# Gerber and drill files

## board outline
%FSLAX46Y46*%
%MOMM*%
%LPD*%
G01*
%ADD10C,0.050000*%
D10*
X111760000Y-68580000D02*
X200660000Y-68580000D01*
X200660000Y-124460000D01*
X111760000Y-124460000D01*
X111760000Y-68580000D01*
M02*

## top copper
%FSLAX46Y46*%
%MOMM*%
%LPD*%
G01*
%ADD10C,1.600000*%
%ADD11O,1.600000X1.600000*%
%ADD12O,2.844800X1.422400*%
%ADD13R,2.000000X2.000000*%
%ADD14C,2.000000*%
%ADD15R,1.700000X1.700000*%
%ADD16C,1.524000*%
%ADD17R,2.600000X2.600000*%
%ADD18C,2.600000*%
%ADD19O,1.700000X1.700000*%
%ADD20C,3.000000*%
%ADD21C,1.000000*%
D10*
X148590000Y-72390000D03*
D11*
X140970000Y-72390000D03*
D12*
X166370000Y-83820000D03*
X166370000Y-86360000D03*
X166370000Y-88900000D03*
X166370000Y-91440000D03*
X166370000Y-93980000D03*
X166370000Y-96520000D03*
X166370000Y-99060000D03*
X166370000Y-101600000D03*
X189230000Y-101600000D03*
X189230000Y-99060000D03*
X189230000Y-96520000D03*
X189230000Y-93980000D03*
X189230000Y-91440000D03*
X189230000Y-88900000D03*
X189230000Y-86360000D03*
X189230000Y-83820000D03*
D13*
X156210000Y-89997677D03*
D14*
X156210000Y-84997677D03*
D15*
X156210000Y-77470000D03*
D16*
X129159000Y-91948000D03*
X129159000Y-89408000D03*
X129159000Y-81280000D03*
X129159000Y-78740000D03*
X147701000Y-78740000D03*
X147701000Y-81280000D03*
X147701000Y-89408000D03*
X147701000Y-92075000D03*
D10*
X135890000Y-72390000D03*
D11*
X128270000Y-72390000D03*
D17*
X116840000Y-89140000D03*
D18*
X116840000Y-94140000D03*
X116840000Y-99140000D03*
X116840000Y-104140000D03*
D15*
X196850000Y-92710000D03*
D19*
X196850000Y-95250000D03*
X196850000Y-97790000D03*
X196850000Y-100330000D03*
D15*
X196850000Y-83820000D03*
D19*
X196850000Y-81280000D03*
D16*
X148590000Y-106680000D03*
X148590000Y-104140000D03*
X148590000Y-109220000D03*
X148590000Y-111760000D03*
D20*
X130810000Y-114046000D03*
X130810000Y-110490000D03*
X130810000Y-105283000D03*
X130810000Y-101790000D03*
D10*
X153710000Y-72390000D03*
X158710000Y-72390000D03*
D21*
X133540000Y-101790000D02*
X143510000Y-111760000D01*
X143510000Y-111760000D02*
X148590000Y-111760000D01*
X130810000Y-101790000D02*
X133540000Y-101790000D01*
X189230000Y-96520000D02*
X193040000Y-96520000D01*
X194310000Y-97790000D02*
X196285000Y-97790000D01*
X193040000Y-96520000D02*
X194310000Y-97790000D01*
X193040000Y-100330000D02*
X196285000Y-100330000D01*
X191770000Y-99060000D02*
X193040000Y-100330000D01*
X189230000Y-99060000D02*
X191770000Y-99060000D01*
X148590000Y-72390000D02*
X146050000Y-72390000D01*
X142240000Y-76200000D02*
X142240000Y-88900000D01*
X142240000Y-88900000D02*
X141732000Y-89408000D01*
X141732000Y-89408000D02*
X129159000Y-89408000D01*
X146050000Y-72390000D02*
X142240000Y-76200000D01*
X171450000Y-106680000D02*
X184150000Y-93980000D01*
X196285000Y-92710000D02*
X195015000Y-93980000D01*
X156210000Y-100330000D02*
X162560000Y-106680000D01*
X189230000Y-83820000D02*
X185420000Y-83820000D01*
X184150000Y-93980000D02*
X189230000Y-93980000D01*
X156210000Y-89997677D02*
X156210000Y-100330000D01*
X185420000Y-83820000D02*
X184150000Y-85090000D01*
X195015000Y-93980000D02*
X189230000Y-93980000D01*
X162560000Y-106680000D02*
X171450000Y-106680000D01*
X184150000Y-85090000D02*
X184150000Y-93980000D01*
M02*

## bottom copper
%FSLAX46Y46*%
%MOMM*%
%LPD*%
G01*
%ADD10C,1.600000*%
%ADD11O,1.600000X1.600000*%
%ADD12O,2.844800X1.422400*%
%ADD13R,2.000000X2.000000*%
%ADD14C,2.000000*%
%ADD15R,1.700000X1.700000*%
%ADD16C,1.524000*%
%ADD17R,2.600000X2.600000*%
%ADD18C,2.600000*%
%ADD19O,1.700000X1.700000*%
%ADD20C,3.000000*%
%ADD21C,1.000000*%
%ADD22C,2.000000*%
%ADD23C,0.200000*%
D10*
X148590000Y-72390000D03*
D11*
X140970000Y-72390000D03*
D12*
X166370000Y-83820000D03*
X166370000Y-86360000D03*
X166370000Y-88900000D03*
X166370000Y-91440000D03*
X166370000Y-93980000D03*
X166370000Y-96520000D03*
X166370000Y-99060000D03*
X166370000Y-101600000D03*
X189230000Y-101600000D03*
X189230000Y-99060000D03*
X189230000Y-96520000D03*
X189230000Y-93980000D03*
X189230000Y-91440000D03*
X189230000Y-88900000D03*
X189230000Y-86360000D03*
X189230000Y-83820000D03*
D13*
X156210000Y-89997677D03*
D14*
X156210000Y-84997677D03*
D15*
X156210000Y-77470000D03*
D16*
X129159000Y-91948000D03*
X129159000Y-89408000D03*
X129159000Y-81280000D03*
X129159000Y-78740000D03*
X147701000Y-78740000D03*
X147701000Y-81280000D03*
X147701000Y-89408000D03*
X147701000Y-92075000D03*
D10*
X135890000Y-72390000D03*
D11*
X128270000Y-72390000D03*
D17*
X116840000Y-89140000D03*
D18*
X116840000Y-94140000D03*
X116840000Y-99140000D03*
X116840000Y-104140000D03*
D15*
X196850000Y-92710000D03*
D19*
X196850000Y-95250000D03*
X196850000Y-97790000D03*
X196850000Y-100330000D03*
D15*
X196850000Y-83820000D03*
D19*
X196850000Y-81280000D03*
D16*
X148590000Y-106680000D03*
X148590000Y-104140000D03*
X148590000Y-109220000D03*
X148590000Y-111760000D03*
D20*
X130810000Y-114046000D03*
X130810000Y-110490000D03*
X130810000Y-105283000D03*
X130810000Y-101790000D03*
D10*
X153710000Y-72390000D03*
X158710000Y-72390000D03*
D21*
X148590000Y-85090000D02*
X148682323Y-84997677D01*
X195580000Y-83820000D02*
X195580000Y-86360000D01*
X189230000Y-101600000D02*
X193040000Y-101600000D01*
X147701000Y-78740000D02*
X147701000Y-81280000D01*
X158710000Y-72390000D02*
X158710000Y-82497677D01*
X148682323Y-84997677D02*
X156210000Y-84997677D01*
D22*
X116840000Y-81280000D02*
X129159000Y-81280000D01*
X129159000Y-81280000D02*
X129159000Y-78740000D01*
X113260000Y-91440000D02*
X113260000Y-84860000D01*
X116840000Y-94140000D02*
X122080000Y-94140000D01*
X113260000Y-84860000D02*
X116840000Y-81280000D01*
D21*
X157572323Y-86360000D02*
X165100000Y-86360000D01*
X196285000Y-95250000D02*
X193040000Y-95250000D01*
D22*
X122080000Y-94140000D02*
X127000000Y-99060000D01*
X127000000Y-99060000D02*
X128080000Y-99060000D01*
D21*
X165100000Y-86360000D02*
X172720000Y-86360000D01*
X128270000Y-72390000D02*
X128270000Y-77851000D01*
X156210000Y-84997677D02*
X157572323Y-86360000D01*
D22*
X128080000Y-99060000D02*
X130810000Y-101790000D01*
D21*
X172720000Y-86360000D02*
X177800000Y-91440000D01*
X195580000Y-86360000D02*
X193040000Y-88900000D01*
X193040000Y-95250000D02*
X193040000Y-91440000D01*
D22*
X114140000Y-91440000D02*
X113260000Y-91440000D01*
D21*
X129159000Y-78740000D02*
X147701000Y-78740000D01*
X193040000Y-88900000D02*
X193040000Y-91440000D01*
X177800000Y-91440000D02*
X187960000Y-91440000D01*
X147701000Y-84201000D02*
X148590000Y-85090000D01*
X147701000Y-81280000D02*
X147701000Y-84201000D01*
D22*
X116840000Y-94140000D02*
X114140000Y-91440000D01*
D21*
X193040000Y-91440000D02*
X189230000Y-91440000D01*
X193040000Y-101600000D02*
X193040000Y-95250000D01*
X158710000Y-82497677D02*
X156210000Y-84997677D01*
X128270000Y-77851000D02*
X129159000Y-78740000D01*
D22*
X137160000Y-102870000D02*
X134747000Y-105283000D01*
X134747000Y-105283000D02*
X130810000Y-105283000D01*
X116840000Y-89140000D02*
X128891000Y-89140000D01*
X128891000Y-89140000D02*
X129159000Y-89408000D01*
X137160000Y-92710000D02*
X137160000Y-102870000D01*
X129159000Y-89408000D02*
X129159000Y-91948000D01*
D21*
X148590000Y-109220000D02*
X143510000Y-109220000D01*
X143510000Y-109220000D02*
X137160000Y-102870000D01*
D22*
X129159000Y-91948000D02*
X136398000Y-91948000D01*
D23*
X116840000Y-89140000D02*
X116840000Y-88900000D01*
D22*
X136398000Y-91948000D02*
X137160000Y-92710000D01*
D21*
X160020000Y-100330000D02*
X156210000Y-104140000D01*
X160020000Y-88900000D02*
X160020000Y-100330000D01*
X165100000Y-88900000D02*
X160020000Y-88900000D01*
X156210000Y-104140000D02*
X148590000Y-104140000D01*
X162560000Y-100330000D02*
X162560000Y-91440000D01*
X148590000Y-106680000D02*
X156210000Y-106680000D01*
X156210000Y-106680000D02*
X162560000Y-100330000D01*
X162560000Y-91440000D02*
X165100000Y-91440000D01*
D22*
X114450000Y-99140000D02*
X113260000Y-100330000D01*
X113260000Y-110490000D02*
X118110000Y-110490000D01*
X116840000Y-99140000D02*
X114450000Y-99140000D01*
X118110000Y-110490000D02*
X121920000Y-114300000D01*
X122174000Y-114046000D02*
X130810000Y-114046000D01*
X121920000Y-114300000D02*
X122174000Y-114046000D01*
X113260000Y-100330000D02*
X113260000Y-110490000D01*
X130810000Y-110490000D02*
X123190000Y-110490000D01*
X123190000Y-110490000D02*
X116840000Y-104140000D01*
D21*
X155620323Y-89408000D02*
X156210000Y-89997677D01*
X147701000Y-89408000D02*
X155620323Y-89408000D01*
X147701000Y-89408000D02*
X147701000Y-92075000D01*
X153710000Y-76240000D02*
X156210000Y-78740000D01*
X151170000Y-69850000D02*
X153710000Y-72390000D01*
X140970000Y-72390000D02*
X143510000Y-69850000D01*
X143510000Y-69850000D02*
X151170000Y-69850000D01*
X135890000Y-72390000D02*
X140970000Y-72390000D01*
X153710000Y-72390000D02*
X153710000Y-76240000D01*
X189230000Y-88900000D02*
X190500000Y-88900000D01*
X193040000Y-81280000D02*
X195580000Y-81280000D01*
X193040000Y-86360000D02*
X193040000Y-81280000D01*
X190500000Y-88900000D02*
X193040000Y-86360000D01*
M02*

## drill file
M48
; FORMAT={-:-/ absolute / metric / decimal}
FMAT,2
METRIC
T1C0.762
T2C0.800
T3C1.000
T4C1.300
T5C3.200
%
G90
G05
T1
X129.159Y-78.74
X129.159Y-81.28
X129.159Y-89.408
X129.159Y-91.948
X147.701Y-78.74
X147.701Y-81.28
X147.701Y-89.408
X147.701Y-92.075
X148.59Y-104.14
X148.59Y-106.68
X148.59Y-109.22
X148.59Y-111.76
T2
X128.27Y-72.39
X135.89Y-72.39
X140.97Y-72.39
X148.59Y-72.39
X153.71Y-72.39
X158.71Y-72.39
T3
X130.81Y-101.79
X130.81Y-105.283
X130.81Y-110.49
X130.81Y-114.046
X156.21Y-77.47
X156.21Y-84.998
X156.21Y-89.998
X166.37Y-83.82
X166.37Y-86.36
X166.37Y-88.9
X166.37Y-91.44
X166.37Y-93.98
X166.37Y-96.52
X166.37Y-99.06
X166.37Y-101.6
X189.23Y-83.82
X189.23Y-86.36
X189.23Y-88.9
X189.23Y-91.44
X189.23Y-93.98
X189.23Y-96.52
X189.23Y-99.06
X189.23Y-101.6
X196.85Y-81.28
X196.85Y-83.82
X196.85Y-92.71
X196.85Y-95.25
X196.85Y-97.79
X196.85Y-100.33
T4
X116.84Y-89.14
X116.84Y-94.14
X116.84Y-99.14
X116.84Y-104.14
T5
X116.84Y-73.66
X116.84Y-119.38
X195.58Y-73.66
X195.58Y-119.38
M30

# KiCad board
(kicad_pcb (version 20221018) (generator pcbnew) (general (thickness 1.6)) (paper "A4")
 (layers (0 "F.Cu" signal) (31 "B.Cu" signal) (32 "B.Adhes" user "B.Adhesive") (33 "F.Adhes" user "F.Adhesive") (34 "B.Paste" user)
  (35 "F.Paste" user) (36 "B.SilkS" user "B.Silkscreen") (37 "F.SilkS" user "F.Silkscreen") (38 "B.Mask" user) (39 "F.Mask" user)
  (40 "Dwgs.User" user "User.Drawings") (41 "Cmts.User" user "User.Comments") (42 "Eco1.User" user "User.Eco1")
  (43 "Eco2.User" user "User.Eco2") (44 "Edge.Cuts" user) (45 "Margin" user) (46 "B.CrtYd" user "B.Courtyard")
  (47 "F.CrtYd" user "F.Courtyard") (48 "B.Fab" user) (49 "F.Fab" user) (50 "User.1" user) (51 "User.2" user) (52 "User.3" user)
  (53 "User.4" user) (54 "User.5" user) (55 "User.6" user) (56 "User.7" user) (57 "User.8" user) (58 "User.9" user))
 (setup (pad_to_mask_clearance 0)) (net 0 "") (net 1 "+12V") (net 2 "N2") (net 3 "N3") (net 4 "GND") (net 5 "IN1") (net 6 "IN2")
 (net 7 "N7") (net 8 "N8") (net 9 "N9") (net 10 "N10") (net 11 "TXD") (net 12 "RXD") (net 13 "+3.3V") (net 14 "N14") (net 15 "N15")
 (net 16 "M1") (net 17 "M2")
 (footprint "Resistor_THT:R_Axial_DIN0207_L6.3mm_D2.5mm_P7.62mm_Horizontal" (layer "F.Cu") (at 148.59 72.39 180)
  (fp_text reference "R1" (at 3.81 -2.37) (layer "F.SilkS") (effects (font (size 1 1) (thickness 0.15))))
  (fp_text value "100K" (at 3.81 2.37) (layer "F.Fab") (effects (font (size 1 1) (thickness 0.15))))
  (pad "1" thru_hole circle (at 0 0 180) (size 1.6 1.6) (drill 0.8) (layers "*.Cu" "*.Mask") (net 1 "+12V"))
  (pad "2" thru_hole oval (at 7.62 0 180) (size 1.6 1.6) (drill 0.8) (layers "*.Cu" "*.Mask") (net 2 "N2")))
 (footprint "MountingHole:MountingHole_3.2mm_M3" (layer "F.Cu") (at 195.58 73.66)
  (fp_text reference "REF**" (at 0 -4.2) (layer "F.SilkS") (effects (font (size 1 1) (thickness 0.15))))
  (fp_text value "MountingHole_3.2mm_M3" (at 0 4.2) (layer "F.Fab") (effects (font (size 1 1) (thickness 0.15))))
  (pad "" np_thru_hole circle (at 0 0) (size 3.2 3.2) (drill 3.2) (layers "F&B.Cu" "*.Mask")))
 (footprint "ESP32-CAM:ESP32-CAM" (layer "F.Cu") (at 177.8 93.98)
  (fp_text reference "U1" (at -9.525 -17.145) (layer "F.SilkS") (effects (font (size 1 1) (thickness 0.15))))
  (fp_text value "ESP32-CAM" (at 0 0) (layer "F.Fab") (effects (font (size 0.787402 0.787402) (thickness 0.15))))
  (pad "P$1" thru_hole oval (at -11.43 -10.16) (size 2.8448 1.4224) (drill 1) (layers "*.Cu" "*.Mask") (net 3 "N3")
   (solder_mask_margin 0.102))
  (pad "P$2" thru_hole oval (at -11.43 -7.62) (size 2.8448 1.4224) (drill 1) (layers "*.Cu" "*.Mask") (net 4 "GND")
   (solder_mask_margin 0.102))
  (pad "P$3" thru_hole oval (at -11.43 -5.08) (size 2.8448 1.4224) (drill 1) (layers "*.Cu" "*.Mask") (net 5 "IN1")
   (solder_mask_margin 0.102))
  (pad "P$4" thru_hole oval (at -11.43 -2.54) (size 2.8448 1.4224) (drill 1) (layers "*.Cu" "*.Mask") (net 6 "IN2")
   (solder_mask_margin 0.102))
  (pad "P$5" thru_hole oval (at -11.43 0) (size 2.8448 1.4224) (drill 1) (layers "*.Cu" "*.Mask") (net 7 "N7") (solder_mask_margin 0.102))
  (pad "P$6" thru_hole oval (at -11.43 2.54) (size 2.8448 1.4224) (drill 1) (layers "*.Cu" "*.Mask") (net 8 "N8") (solder_mask_margin 0.102))
  (pad "P$7" thru_hole oval (at -11.43 5.08) (size 2.8448 1.4224) (drill 1) (layers "*.Cu" "*.Mask") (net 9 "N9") (solder_mask_margin 0.102))
  (pad "P$8" thru_hole oval (at -11.43 7.62) (size 2.8448 1.4224) (drill 1) (layers "*.Cu" "*.Mask") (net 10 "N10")
   (solder_mask_margin 0.102))
  (pad "P$9" thru_hole oval (at 11.43 7.62) (size 2.8448 1.4224) (drill 1) (layers "*.Cu" "*.Mask") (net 4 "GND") (solder_mask_margin 0.102))
  (pad "P$10" thru_hole oval (at 11.43 5.08) (size 2.8448 1.4224) (drill 1) (layers "*.Cu" "*.Mask") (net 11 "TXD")
   (solder_mask_margin 0.102))
  (pad "P$11" thru_hole oval (at 11.43 2.54) (size 2.8448 1.4224) (drill 1) (layers "*.Cu" "*.Mask") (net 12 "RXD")
   (solder_mask_margin 0.102))
  (pad "P$12" thru_hole oval (at 11.43 0) (size 2.8448 1.4224) (drill 1) (layers "*.Cu" "*.Mask") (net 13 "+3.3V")
   (solder_mask_margin 0.102))
  (pad "P$13" thru_hole oval (at 11.43 -2.54) (size 2.8448 1.4224) (drill 1) (layers "*.Cu" "*.Mask") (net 4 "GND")
   (solder_mask_margin 0.102))
  (pad "P$14" thru_hole oval (at 11.43 -5.08) (size 2.8448 1.4224) (drill 1) (layers "*.Cu" "*.Mask") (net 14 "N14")
   (solder_mask_margin 0.102))
  (pad "P$15" thru_hole oval (at 11.43 -7.62) (size 2.8448 1.4224) (drill 1) (layers "*.Cu" "*.Mask") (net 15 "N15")
   (solder_mask_margin 0.102))
  (pad "P$16" thru_hole oval (at 11.43 -10.16) (size 2.8448 1.4224) (drill 1) (layers "*.Cu" "*.Mask") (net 13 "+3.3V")
   (solder_mask_margin 0.102)))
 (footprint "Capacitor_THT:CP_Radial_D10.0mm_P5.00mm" (layer "F.Cu") (at 156.21 89.997677 90)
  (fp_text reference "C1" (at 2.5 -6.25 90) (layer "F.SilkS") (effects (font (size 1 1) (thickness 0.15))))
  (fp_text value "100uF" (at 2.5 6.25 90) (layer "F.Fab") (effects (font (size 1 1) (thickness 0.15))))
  (pad "1" thru_hole rect (at 0 0 90) (size 2 2) (drill 1) (layers "*.Cu" "*.Mask") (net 13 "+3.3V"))
  (pad "2" thru_hole circle (at 5 0 90) (size 2 2) (drill 1) (layers "*.Cu" "*.Mask") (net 4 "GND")))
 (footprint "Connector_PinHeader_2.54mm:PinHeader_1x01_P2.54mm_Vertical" (layer "F.Cu") (at 156.21 77.47)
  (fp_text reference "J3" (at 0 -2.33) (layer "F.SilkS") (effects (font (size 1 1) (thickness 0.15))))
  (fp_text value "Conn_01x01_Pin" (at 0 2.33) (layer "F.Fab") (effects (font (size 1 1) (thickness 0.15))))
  (pad "1" thru_hole rect (at 0 0) (size 1.7 1.7) (drill 1) (layers "*.Cu" "*.Mask") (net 2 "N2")))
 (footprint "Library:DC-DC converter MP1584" (layer "F.Cu") (at 129.159 91.948)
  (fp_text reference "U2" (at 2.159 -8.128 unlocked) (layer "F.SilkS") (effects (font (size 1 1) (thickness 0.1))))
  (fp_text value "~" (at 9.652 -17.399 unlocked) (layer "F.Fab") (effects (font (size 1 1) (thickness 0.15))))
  (pad "1" thru_hole circle (at 0 0) (size 1.524 1.524) (drill 0.762) (layers "*.Cu" "*.Mask") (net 1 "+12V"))
  (pad "2" thru_hole circle (at 0 -2.54) (size 1.524 1.524) (drill 0.762) (layers "*.Cu" "*.Mask") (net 1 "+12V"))
  (pad "3" thru_hole circle (at 0 -10.668) (size 1.524 1.524) (drill 0.762) (layers "*.Cu" "*.Mask") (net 4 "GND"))
  (pad "4" thru_hole circle (at 0 -13.208) (size 1.524 1.524) (drill 0.762) (layers "*.Cu" "*.Mask") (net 4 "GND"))
  (pad "5" thru_hole circle (at 18.542 -13.208) (size 1.524 1.524) (drill 0.762) (layers "*.Cu" "*.Mask") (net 4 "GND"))
  (pad "6" thru_hole circle (at 18.542 -10.668) (size 1.524 1.524) (drill 0.762) (layers "*.Cu" "*.Mask") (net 4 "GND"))
  (pad "7" thru_hole circle (at 18.542 -2.54) (size 1.524 1.524) (drill 0.762) (layers "*.Cu" "*.Mask") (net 13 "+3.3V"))
  (pad "8" thru_hole circle (at 18.542 0.127) (size 1.524 1.524) (drill 0.762) (layers "*.Cu" "*.Mask") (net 13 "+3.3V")))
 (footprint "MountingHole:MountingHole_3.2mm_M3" (layer "F.Cu") (at 116.84 119.38)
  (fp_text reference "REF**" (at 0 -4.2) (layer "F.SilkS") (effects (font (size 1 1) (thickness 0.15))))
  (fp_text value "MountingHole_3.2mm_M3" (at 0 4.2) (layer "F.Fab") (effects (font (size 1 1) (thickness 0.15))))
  (pad "" np_thru_hole circle (at 0 0) (size 3.2 3.2) (drill 3.2) (layers "F&B.Cu" "*.Mask")))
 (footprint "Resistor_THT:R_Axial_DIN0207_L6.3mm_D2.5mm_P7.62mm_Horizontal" (layer "F.Cu") (at 135.89 72.39 180)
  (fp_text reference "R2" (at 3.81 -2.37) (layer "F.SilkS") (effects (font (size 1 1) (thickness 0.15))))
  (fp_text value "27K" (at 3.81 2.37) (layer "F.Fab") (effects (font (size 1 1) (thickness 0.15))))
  (pad "1" thru_hole circle (at 0 0 180) (size 1.6 1.6) (drill 0.8) (layers "*.Cu" "*.Mask") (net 2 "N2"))
  (pad "2" thru_hole oval (at 7.62 0 180) (size 1.6 1.6) (drill 0.8) (layers "*.Cu" "*.Mask") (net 4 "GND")))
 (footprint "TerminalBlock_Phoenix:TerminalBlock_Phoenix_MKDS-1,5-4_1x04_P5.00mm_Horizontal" (layer "F.Cu") (at 116.84 89.14 -90)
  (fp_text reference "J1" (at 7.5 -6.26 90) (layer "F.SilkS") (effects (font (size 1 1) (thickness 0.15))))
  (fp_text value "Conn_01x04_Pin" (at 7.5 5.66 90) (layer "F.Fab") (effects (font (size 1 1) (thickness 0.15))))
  (pad "1" thru_hole rect (at 0 0 270) (size 2.6 2.6) (drill 1.3) (layers "*.Cu" "*.Mask") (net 1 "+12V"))
  (pad "2" thru_hole circle (at 5 0 270) (size 2.6 2.6) (drill 1.3) (layers "*.Cu" "*.Mask") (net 4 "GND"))
  (pad "3" thru_hole circle (at 10 0 270) (size 2.6 2.6) (drill 1.3) (layers "*.Cu" "*.Mask") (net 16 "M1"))
  (pad "4" thru_hole circle (at 15 0 270) (size 2.6 2.6) (drill 1.3) (layers "*.Cu" "*.Mask") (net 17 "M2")))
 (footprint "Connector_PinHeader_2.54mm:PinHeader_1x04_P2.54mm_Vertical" (layer "F.Cu") (at 196.85 92.71)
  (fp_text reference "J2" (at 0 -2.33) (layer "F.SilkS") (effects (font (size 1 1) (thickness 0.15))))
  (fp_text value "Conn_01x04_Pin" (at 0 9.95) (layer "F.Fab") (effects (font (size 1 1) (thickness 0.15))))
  (pad "1" thru_hole rect (at 0 0) (size 1.7 1.7) (drill 1) (layers "*.Cu" "*.Mask") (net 13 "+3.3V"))
  (pad "2" thru_hole oval (at 0 2.54) (size 1.7 1.7) (drill 1) (layers "*.Cu" "*.Mask") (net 4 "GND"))
  (pad "3" thru_hole oval (at 0 5.08) (size 1.7 1.7) (drill 1) (layers "*.Cu" "*.Mask") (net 12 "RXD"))
  (pad "4" thru_hole oval (at 0 7.62) (size 1.7 1.7) (drill 1) (layers "*.Cu" "*.Mask") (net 11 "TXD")))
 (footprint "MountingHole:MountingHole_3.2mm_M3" (layer "F.Cu") (at 116.84 73.66)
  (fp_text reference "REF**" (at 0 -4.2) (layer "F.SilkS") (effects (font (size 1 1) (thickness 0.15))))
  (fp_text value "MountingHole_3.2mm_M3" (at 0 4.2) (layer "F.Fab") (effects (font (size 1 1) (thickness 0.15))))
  (pad "" np_thru_hole circle (at 0 0) (size 3.2 3.2) (drill 3.2) (layers "*.Cu" "*.Mask")))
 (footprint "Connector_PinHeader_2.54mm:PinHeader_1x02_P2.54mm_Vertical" (layer "F.Cu") (at 196.85 83.82 180)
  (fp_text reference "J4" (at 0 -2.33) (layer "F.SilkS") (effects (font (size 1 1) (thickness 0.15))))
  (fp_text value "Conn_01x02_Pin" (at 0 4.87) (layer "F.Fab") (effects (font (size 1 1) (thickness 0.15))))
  (pad "1" thru_hole rect (at 0 0 180) (size 1.7 1.7) (drill 1) (layers "*.Cu" "*.Mask") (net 4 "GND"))
  (pad "2" thru_hole oval (at 0 2.54 180) (size 1.7 1.7) (drill 1) (layers "*.Cu" "*.Mask") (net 14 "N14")))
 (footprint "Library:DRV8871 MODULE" (layer "F.Cu") (at 151.13 97.79 180)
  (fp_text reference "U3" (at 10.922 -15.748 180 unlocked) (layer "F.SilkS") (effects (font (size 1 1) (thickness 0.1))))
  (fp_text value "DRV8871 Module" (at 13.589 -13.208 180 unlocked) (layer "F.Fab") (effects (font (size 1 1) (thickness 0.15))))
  (pad "1" thru_hole circle (at 2.54 -8.89 180) (size 1.524 1.524) (drill 0.762) (layers "*.Cu" "*.Mask") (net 6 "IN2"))
  (pad "2" thru_hole circle (at 2.54 -6.35 180) (size 1.524 1.524) (drill 0.762) (layers "*.Cu" "*.Mask") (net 5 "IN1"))
  (pad "3" thru_hole circle (at 2.54 -11.43 180) (size 1.524 1.524) (drill 0.762) (layers "*.Cu" "*.Mask") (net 1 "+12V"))
  (pad "4" thru_hole circle (at 2.54 -13.97 180) (size 1.524 1.524) (drill 0.762) (layers "*.Cu" "*.Mask") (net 4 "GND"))
  (pad "5" thru_hole circle (at 20.32 -16.256 180) (size 3 3) (drill 1) (layers "*.Cu" "*.Mask") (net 16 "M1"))
  (pad "6" thru_hole circle (at 20.32 -12.7 180) (size 3 3) (drill 1) (layers "*.Cu" "*.Mask") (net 17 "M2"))
  (pad "7" thru_hole circle (at 20.32 -7.493 180) (size 3 3) (drill 1) (layers "*.Cu" "*.Mask") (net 1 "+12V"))
  (pad "8" thru_hole circle (at 20.32 -4 180) (size 3 3) (drill 1) (layers "*.Cu" "*.Mask") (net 4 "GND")))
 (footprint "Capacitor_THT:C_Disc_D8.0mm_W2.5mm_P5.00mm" (layer "F.Cu") (at 153.71 72.39)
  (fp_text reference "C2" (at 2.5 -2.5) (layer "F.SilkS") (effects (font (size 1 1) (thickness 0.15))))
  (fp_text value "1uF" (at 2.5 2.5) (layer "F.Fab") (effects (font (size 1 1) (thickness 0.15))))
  (pad "1" thru_hole circle (at 0 0) (size 1.6 1.6) (drill 0.8) (layers "*.Cu" "*.Mask") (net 2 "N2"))
  (pad "2" thru_hole circle (at 5 0) (size 1.6 1.6) (drill 0.8) (layers "*.Cu" "*.Mask") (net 4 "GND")))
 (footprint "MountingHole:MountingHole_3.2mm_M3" (layer "F.Cu") (at 195.58 119.38)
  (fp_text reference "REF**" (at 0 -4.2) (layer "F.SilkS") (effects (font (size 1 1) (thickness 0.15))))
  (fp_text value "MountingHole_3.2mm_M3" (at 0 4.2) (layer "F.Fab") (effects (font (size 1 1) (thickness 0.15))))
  (pad "" np_thru_hole circle (at 0 0) (size 3.2 3.2) (drill 3.2) (layers "F&B.Cu" "*.Mask")))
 (gr_rect (start 111.76 68.58) (end 200.66 124.46) (stroke (width 0.05) (type default)) (fill none) (layer "Edge.Cuts"))
 (segment (start 133.54 101.79) (end 143.51 111.76) (width 1) (layer "F.Cu") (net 4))
 (segment (start 143.51 111.76) (end 148.59 111.76) (width 1) (layer "F.Cu") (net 4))
 (segment (start 130.81 101.79) (end 133.54 101.79) (width 1) (layer "F.Cu") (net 4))
 (segment (start 148.59 85.09) (end 148.682323 84.997677) (width 1) (layer "B.Cu") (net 4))
 (segment (start 195.58 83.82) (end 195.58 86.36) (width 1) (layer "B.Cu") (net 4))
 (segment (start 189.23 101.6) (end 193.04 101.6) (width 1) (layer "B.Cu") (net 4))
 (segment (start 147.701 78.74) (end 147.701 81.28) (width 1) (layer "B.Cu") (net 4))
 (segment (start 158.71 72.39) (end 158.71 82.497677) (width 1) (layer "B.Cu") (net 4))
 (segment (start 148.682323 84.997677) (end 156.21 84.997677) (width 1) (layer "B.Cu") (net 4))
 (segment (start 116.84 81.28) (end 129.159 81.28) (width 2) (layer "B.Cu") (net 4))
 (segment (start 129.159 81.28) (end 129.159 78.74) (width 2) (layer "B.Cu") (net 4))
 (segment (start 113.26 91.44) (end 113.26 84.86) (width 2) (layer "B.Cu") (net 4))
 (segment (start 116.84 94.14) (end 122.08 94.14) (width 2) (layer "B.Cu") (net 4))
 (segment (start 113.26 84.86) (end 116.84 81.28) (width 2) (layer "B.Cu") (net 4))
 (segment (start 157.572323 86.36) (end 165.1 86.36) (width 1) (layer "B.Cu") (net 4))
 (segment (start 196.285 95.25) (end 193.04 95.25) (width 1) (layer "B.Cu") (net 4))
 (segment (start 122.08 94.14) (end 127 99.06) (width 2) (layer "B.Cu") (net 4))
 (segment (start 127 99.06) (end 128.08 99.06) (width 2) (layer "B.Cu") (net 4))
 (segment (start 165.1 86.36) (end 172.72 86.36) (width 1) (layer "B.Cu") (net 4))
 (segment (start 128.27 72.39) (end 128.27 77.851) (width 1) (layer "B.Cu") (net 4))
 (segment (start 156.21 84.997677) (end 157.572323 86.36) (width 1) (layer "B.Cu") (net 4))
 (segment (start 128.08 99.06) (end 130.81 101.79) (width 2) (layer "B.Cu") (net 4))
 (segment (start 172.72 86.36) (end 177.8 91.44) (width 1) (layer "B.Cu") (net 4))
 (segment (start 195.58 86.36) (end 193.04 88.9) (width 1) (layer "B.Cu") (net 4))
 (segment (start 193.04 95.25) (end 193.04 91.44) (width 1) (layer "B.Cu") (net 4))
 (segment (start 114.14 91.44) (end 113.26 91.44) (width 2) (layer "B.Cu") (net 4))
 (segment (start 129.159 78.74) (end 147.701 78.74) (width 1) (layer "B.Cu") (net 4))
 (segment (start 193.04 88.9) (end 193.04 91.44) (width 1) (layer "B.Cu") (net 4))
 (segment (start 177.8 91.44) (end 187.96 91.44) (width 1) (layer "B.Cu") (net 4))
 (segment (start 147.701 84.201) (end 148.59 85.09) (width 1) (layer "B.Cu") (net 4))
 (segment (start 147.701 81.28) (end 147.701 84.201) (width 1) (layer "B.Cu") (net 4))
 (segment (start 116.84 94.14) (end 114.14 91.44) (width 2) (layer "B.Cu") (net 4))
 (segment (start 193.04 91.44) (end 189.23 91.44) (width 1) (layer "B.Cu") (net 4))
 (segment (start 193.04 101.6) (end 193.04 95.25) (width 1) (layer "B.Cu") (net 4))
 (segment (start 158.71 82.497677) (end 156.21 84.997677) (width 1) (layer "B.Cu") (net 4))
 (segment (start 128.27 77.851) (end 129.159 78.74) (width 1) (layer "B.Cu") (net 4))
 (segment (start 189.23 96.52) (end 193.04 96.52) (width 1) (layer "F.Cu") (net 12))
 (segment (start 194.31 97.79) (end 196.285 97.79) (width 1) (layer "F.Cu") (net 12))
 (segment (start 193.04 96.52) (end 194.31 97.79) (width 1) (layer "F.Cu") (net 12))
 (segment (start 193.04 100.33) (end 196.285 100.33) (width 1) (layer "F.Cu") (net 11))
 (segment (start 191.77 99.06) (end 193.04 100.33) (width 1) (layer "F.Cu") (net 11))
 (segment (start 189.23 99.06) (end 191.77 99.06) (width 1) (layer "F.Cu") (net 11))
 (segment (start 148.59 72.39) (end 146.05 72.39) (width 1) (layer "F.Cu") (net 1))
 (segment (start 142.24 76.2) (end 142.24 88.9) (width 1) (layer "F.Cu") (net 1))
 (segment (start 142.24 88.9) (end 141.732 89.408) (width 1) (layer "F.Cu") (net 1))
 (segment (start 141.732 89.408) (end 129.159 89.408) (width 1) (layer "F.Cu") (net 1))
 (segment (start 146.05 72.39) (end 142.24 76.2) (width 1) (layer "F.Cu") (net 1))
 (segment (start 137.16 102.87) (end 134.747 105.283) (width 2) (layer "B.Cu") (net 1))
 (segment (start 134.747 105.283) (end 130.81 105.283) (width 2) (layer "B.Cu") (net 1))
 (segment (start 116.84 89.14) (end 128.891 89.14) (width 2) (layer "B.Cu") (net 1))
 (segment (start 128.891 89.14) (end 129.159 89.408) (width 2) (layer "B.Cu") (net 1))
 (segment (start 137.16 92.71) (end 137.16 102.87) (width 2) (layer "B.Cu") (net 1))
 (segment (start 129.159 89.408) (end 129.159 91.948) (width 2) (layer "B.Cu") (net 1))
 (segment (start 148.59 109.22) (end 143.51 109.22) (width 1) (layer "B.Cu") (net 1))
 (segment (start 143.51 109.22) (end 137.16 102.87) (width 1) (layer "B.Cu") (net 1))
 (segment (start 129.159 91.948) (end 136.398 91.948) (width 2) (layer "B.Cu") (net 1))
 (segment (start 116.84 89.14) (end 116.84 88.9) (width 0.2) (layer "B.Cu") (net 1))
 (segment (start 136.398 91.948) (end 137.16 92.71) (width 2) (layer "B.Cu") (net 1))
 (segment (start 160.02 100.33) (end 156.21 104.14) (width 1) (layer "B.Cu") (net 5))
 (segment (start 160.02 88.9) (end 160.02 100.33) (width 1) (layer "B.Cu") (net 5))
 (segment (start 165.1 88.9) (end 160.02 88.9) (width 1) (layer "B.Cu") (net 5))
 (segment (start 156.21 104.14) (end 148.59 104.14) (width 1) (layer "B.Cu") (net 5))
 (segment (start 162.56 100.33) (end 162.56 91.44) (width 1) (layer "B.Cu") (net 6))
 (segment (start 148.59 106.68) (end 156.21 106.68) (width 1) (layer "B.Cu") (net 6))
 (segment (start 156.21 106.68) (end 162.56 100.33) (width 1) (layer "B.Cu") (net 6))
 (segment (start 162.56 91.44) (end 165.1 91.44) (width 1) (layer "B.Cu") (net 6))
 (segment (start 114.45 99.14) (end 113.26 100.33) (width 2) (layer "B.Cu") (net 16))
 (segment (start 113.26 110.49) (end 118.11 110.49) (width 2) (layer "B.Cu") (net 16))
 (segment (start 116.84 99.14) (end 114.45 99.14) (width 2) (layer "B.Cu") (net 16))
 (segment (start 118.11 110.49) (end 121.92 114.3) (width 2) (layer "B.Cu") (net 16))
 (segment (start 122.174 114.046) (end 130.81 114.046) (width 2) (layer "B.Cu") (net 16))
 (segment (start 121.92 114.3) (end 122.174 114.046) (width 2) (layer "B.Cu") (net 16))
 (segment (start 113.26 100.33) (end 113.26 110.49) (width 2) (layer "B.Cu") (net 16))
 (segment (start 130.81 110.49) (end 123.19 110.49) (width 2) (layer "B.Cu") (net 17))
 (segment (start 123.19 110.49) (end 116.84 104.14) (width 2) (layer "B.Cu") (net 17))
 (segment (start 171.45 106.68) (end 184.15 93.98) (width 1) (layer "F.Cu") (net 13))
 (segment (start 196.285 92.71) (end 195.015 93.98) (width 1) (layer "F.Cu") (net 13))
 (segment (start 156.21 100.33) (end 162.56 106.68) (width 1) (layer "F.Cu") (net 13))
 (segment (start 189.23 83.82) (end 185.42 83.82) (width 1) (layer "F.Cu") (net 13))
 (segment (start 184.15 93.98) (end 189.23 93.98) (width 1) (layer "F.Cu") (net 13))
 (segment (start 156.21 89.997677) (end 156.21 100.33) (width 1) (layer "F.Cu") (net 13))
 (segment (start 185.42 83.82) (end 184.15 85.09) (width 1) (layer "F.Cu") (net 13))
 (segment (start 195.015 93.98) (end 189.23 93.98) (width 1) (layer "F.Cu") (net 13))
 (segment (start 162.56 106.68) (end 171.45 106.68) (width 1) (layer "F.Cu") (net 13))
 (segment (start 184.15 85.09) (end 184.15 93.98) (width 1) (layer "F.Cu") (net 13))
 (segment (start 155.620323 89.408) (end 156.21 89.997677) (width 1) (layer "B.Cu") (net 13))
 (segment (start 147.701 89.408) (end 155.620323 89.408) (width 1) (layer "B.Cu") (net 13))
 (segment (start 147.701 89.408) (end 147.701 92.075) (width 1) (layer "B.Cu") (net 13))
 (segment (start 153.71 76.24) (end 156.21 78.74) (width 1) (layer "B.Cu") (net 2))
 (segment (start 151.17 69.85) (end 153.71 72.39) (width 1) (layer "B.Cu") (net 2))
 (segment (start 140.97 72.39) (end 143.51 69.85) (width 1) (layer "B.Cu") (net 2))
 (segment (start 143.51 69.85) (end 151.17 69.85) (width 1) (layer "B.Cu") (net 2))
 (segment (start 135.89 72.39) (end 140.97 72.39) (width 1) (layer "B.Cu") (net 2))
 (segment (start 153.71 72.39) (end 153.71 76.24) (width 1) (layer "B.Cu") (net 2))
 (segment (start 189.23 88.9) (end 190.5 88.9) (width 1) (layer "B.Cu") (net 14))
 (segment (start 193.04 81.28) (end 195.58 81.28) (width 1) (layer "B.Cu") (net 14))
 (segment (start 193.04 86.36) (end 193.04 81.28) (width 1) (layer "B.Cu") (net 14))
 (segment (start 190.5 88.9) (end 193.04 86.36) (width 1) (layer "B.Cu") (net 14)))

